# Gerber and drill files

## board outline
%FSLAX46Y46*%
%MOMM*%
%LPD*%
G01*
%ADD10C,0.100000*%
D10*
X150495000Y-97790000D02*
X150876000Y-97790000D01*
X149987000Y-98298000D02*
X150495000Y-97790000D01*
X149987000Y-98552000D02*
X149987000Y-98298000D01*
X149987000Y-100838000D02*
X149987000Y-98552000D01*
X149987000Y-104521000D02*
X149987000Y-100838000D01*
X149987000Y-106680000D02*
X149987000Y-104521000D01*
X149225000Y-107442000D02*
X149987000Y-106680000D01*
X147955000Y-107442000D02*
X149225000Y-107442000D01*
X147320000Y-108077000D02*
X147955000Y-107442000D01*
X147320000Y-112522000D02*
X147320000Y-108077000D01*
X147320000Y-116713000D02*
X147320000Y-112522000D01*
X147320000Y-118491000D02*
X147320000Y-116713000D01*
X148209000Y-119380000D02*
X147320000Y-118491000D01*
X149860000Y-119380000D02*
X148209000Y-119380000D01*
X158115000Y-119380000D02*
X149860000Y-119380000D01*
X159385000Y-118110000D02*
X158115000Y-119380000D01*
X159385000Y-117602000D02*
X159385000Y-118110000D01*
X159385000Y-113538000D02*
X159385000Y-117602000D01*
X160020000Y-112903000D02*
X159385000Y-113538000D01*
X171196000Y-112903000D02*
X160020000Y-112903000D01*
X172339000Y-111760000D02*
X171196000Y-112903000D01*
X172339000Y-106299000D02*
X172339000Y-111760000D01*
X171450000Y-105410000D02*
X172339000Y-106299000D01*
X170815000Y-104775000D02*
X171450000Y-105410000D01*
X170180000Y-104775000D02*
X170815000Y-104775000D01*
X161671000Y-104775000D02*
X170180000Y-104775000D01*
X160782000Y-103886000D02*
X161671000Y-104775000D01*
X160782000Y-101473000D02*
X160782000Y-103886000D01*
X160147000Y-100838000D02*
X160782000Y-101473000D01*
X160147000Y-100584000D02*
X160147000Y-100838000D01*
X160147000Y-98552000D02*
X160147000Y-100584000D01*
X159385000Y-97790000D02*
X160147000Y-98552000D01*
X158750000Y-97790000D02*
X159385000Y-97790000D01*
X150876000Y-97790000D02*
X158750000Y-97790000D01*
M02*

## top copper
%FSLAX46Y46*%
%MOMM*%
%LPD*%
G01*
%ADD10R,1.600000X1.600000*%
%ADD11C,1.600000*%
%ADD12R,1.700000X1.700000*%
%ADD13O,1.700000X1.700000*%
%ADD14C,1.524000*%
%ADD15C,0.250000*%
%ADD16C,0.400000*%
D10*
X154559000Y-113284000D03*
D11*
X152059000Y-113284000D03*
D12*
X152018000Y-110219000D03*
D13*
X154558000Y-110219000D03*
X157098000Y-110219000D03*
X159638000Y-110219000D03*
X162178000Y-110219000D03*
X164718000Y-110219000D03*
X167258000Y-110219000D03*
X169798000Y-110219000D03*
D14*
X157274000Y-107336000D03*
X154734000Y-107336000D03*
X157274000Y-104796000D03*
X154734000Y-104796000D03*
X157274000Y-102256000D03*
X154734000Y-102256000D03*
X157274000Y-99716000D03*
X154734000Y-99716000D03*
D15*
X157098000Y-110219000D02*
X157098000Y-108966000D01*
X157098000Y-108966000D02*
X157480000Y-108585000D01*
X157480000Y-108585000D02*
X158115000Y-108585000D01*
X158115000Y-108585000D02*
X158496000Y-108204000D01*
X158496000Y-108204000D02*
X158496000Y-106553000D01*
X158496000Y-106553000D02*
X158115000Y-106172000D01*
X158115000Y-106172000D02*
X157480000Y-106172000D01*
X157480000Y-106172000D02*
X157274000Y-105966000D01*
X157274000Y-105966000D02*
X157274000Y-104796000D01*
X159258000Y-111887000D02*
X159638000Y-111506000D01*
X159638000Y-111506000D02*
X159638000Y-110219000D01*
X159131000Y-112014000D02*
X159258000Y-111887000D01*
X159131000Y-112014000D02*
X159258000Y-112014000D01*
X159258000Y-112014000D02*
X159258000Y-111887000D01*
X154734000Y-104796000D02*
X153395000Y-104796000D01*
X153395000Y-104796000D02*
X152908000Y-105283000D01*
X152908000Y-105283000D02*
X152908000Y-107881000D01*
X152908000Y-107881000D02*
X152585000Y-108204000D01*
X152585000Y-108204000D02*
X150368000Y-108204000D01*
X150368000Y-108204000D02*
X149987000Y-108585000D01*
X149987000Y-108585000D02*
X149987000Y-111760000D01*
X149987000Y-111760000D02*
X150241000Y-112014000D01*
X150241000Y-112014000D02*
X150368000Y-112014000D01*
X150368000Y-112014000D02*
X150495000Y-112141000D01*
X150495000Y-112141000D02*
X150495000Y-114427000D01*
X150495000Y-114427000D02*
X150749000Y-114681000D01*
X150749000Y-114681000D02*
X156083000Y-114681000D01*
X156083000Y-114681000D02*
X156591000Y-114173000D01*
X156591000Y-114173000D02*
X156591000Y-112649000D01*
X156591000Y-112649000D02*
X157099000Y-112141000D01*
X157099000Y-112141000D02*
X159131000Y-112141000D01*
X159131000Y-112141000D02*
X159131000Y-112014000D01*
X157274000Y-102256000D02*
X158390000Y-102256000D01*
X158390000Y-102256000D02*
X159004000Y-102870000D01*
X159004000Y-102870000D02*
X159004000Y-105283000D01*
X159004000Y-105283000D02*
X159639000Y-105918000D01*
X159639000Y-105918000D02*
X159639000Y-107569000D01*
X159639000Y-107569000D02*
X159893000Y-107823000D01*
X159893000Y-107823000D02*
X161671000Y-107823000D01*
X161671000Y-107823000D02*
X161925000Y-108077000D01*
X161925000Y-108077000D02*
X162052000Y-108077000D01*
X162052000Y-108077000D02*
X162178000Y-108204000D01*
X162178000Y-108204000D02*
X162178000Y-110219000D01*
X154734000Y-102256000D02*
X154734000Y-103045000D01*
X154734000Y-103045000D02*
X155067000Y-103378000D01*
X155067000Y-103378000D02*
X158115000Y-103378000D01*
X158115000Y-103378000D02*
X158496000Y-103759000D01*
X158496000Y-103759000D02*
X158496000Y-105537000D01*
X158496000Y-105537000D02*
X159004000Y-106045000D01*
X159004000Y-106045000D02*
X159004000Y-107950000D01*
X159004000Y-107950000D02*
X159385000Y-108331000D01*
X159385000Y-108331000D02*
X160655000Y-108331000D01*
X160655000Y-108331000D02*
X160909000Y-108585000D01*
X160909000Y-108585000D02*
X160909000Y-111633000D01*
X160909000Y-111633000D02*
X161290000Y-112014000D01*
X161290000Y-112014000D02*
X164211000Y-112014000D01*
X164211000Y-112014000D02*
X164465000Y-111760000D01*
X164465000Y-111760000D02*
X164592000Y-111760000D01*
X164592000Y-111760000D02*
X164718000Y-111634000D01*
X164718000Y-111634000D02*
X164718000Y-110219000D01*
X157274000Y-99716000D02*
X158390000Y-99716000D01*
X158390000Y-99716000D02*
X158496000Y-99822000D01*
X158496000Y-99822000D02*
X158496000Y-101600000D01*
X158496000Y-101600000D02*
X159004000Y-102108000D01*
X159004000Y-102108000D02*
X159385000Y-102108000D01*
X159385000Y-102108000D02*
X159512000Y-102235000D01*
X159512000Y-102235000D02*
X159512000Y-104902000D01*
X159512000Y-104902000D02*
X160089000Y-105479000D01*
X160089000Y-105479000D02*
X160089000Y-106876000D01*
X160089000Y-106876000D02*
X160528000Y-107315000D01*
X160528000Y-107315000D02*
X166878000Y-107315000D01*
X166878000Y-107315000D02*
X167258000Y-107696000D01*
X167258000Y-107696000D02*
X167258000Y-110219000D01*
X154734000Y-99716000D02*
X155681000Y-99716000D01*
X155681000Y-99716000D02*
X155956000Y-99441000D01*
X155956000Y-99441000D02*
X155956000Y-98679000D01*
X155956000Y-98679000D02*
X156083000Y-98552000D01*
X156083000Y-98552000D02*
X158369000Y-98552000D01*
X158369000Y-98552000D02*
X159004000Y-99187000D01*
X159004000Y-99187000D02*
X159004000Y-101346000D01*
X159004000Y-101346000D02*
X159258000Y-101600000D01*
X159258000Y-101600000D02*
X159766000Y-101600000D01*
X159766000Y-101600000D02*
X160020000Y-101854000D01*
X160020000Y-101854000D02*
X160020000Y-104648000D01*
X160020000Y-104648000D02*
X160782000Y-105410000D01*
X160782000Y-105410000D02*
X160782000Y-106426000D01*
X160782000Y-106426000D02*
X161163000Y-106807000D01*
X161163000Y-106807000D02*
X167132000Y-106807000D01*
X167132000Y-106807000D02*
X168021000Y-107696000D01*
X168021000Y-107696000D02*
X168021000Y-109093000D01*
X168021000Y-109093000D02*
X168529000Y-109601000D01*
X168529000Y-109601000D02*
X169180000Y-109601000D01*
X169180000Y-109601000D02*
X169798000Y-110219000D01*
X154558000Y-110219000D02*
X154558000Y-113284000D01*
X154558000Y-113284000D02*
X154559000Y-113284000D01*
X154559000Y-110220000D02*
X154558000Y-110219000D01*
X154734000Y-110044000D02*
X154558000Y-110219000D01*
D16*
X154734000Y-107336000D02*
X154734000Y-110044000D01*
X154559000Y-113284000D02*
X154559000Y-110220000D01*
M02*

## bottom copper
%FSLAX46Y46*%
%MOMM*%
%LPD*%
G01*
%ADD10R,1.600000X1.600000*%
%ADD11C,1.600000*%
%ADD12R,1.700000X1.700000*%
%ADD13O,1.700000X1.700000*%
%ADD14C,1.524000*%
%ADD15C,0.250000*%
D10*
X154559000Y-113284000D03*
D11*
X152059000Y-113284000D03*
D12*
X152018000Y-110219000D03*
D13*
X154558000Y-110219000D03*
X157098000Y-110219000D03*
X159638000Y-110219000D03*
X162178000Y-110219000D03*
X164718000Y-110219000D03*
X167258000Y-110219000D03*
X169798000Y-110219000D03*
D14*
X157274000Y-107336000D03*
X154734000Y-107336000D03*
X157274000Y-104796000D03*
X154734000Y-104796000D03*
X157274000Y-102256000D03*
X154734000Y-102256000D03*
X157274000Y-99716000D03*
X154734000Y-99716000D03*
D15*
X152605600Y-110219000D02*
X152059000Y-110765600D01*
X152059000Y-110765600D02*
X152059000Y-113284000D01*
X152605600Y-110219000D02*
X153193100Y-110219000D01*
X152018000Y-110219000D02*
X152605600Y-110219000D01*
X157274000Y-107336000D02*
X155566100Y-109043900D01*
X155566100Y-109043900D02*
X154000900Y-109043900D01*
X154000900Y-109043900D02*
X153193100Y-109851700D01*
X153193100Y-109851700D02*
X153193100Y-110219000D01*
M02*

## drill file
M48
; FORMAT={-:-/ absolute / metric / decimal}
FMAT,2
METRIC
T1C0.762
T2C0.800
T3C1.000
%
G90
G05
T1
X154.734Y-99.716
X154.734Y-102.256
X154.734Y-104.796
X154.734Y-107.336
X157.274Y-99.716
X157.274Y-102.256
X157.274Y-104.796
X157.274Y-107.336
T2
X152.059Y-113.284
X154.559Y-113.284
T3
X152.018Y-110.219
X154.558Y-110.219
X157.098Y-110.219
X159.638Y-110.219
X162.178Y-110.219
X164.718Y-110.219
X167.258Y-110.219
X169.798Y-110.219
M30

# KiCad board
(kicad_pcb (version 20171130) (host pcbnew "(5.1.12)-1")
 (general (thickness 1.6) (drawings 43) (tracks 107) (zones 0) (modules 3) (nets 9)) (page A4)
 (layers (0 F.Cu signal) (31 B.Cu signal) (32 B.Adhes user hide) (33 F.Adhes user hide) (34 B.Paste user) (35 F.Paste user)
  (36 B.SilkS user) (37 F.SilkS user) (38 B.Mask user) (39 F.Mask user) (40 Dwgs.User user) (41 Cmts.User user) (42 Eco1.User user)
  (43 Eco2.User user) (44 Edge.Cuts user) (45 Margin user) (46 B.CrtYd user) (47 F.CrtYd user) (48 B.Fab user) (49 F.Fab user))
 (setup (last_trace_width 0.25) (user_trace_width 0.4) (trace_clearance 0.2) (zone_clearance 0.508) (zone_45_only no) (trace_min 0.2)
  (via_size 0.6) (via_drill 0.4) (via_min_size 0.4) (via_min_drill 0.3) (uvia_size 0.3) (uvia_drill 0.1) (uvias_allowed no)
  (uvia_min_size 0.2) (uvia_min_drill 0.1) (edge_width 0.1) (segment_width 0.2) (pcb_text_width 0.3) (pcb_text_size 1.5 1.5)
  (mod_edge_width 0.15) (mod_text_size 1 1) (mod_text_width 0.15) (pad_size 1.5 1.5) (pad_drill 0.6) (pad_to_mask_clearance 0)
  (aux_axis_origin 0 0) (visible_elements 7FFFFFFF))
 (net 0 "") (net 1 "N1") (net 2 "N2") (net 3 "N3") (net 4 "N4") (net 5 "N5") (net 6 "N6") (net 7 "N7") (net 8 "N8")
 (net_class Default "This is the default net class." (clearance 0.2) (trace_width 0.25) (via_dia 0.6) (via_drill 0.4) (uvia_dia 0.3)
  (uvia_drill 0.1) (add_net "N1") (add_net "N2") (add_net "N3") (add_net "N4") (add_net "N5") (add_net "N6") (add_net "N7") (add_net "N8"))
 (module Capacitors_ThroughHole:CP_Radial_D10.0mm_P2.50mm (layer F.Cu) (at 154.559 113.284 180)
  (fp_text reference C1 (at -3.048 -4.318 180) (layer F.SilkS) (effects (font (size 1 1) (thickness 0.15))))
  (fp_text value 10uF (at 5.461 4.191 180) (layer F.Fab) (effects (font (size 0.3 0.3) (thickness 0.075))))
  (pad 1 thru_hole rect (at 0 0 180) (size 1.6 1.6) (drill 0.8) (layers *.Cu *.Mask) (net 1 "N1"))
  (pad 2 thru_hole circle (at 2.5 0 180) (size 1.6 1.6) (drill 0.8) (layers *.Cu *.Mask) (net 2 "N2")))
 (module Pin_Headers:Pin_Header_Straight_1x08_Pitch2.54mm (layer F.Cu) (at 152.018 110.219 90)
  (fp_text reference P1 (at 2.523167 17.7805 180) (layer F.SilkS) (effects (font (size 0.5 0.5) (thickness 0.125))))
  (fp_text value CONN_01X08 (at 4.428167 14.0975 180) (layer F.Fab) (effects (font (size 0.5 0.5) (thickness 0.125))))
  (pad 1 thru_hole rect (at 0 0 90) (size 1.7 1.7) (drill 1) (layers *.Cu *.Mask) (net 2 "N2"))
  (pad 2 thru_hole oval (at 0 2.54 90) (size 1.7 1.7) (drill 1) (layers *.Cu *.Mask) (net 1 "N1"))
  (pad 3 thru_hole oval (at 0 5.08 90) (size 1.7 1.7) (drill 1) (layers *.Cu *.Mask) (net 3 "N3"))
  (pad 4 thru_hole oval (at 0 7.62 90) (size 1.7 1.7) (drill 1) (layers *.Cu *.Mask) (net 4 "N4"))
  (pad 5 thru_hole oval (at 0 10.16 90) (size 1.7 1.7) (drill 1) (layers *.Cu *.Mask) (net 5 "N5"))
  (pad 6 thru_hole oval (at 0 12.7 90) (size 1.7 1.7) (drill 1) (layers *.Cu *.Mask) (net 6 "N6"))
  (pad 7 thru_hole oval (at 0 15.24 90) (size 1.7 1.7) (drill 1) (layers *.Cu *.Mask) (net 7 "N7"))
  (pad 8 thru_hole oval (at 0 17.78 90) (size 1.7 1.7) (drill 1) (layers *.Cu *.Mask) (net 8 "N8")))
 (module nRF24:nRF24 (layer F.Cu) (at 154.734 103.78)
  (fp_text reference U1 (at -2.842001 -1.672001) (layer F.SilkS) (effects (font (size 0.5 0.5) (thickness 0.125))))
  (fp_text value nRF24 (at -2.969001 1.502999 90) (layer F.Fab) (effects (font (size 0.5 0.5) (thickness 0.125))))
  (pad 1 thru_hole circle (at 2.54 3.556) (size 1.524 1.524) (drill 0.762) (layers *.Cu *.Mask) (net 2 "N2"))
  (pad 2 thru_hole circle (at 0 3.556) (size 1.524 1.524) (drill 0.762) (layers *.Cu *.Mask) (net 1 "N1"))
  (pad 3 thru_hole circle (at 2.54 1.016) (size 1.524 1.524) (drill 0.762) (layers *.Cu *.Mask) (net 3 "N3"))
  (pad 4 thru_hole circle (at 0 1.016) (size 1.524 1.524) (drill 0.762) (layers *.Cu *.Mask) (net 4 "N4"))
  (pad 5 thru_hole circle (at 2.54 -1.524) (size 1.524 1.524) (drill 0.762) (layers *.Cu *.Mask) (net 5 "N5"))
  (pad 6 thru_hole circle (at 0 -1.524) (size 1.524 1.524) (drill 0.762) (layers *.Cu *.Mask) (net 6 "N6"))
  (pad 7 thru_hole circle (at 2.54 -4.064) (size 1.524 1.524) (drill 0.762) (layers *.Cu *.Mask) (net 7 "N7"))
  (pad 8 thru_hole circle (at 0 -4.064) (size 1.524 1.524) (drill 0.762) (layers *.Cu *.Mask) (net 8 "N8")))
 (gr_line (start 150.495 97.79) (end 150.876 97.79) (angle 90) (layer Edge.Cuts) (width 0.1))
 (gr_line (start 149.987 98.298) (end 150.495 97.79) (angle 90) (layer Edge.Cuts) (width 0.1))
 (gr_line (start 149.987 98.552) (end 149.987 98.298) (angle 90) (layer Edge.Cuts) (width 0.1))
 (gr_line (start 149.987 100.838) (end 149.987 98.552) (angle 90) (layer Edge.Cuts) (width 0.1))
 (gr_line (start 149.987 104.521) (end 149.987 100.838) (angle 90) (layer Edge.Cuts) (width 0.1))
 (gr_line (start 149.987 106.68) (end 149.987 104.521) (angle 90) (layer Edge.Cuts) (width 0.1))
 (gr_line (start 149.225 107.442) (end 149.987 106.68) (angle 90) (layer Edge.Cuts) (width 0.1))
 (gr_line (start 147.955 107.442) (end 149.225 107.442) (angle 90) (layer Edge.Cuts) (width 0.1))
 (gr_line (start 147.32 108.077) (end 147.955 107.442) (angle 90) (layer Edge.Cuts) (width 0.1))
 (gr_line (start 147.32 112.522) (end 147.32 108.077) (angle 90) (layer Edge.Cuts) (width 0.1))
 (gr_line (start 147.32 116.713) (end 147.32 112.522) (angle 90) (layer Edge.Cuts) (width 0.1))
 (gr_line (start 147.32 118.491) (end 147.32 116.713) (angle 90) (layer Edge.Cuts) (width 0.1))
 (gr_line (start 148.209 119.38) (end 147.32 118.491) (angle 90) (layer Edge.Cuts) (width 0.1))
 (gr_line (start 149.86 119.38) (end 148.209 119.38) (angle 90) (layer Edge.Cuts) (width 0.1))
 (gr_line (start 158.115 119.38) (end 149.86 119.38) (angle 90) (layer Edge.Cuts) (width 0.1))
 (gr_line (start 159.385 118.11) (end 158.115 119.38) (angle 90) (layer Edge.Cuts) (width 0.1))
 (gr_line (start 159.385 117.602) (end 159.385 118.11) (angle 90) (layer Edge.Cuts) (width 0.1))
 (gr_line (start 159.385 113.538) (end 159.385 117.602) (angle 90) (layer Edge.Cuts) (width 0.1))
 (gr_line (start 160.02 112.903) (end 159.385 113.538) (angle 90) (layer Edge.Cuts) (width 0.1))
 (gr_line (start 171.196 112.903) (end 160.02 112.903) (angle 90) (layer Edge.Cuts) (width 0.1))
 (gr_line (start 172.339 111.76) (end 171.196 112.903) (angle 90) (layer Edge.Cuts) (width 0.1))
 (gr_line (start 172.339 106.299) (end 172.339 111.76) (angle 90) (layer Edge.Cuts) (width 0.1))
 (gr_line (start 171.45 105.41) (end 172.339 106.299) (angle 90) (layer Edge.Cuts) (width 0.1))
 (gr_line (start 170.815 104.775) (end 171.45 105.41) (angle 90) (layer Edge.Cuts) (width 0.1))
 (gr_line (start 170.18 104.775) (end 170.815 104.775) (angle 90) (layer Edge.Cuts) (width 0.1))
 (gr_line (start 161.671 104.775) (end 170.18 104.775) (angle 90) (layer Edge.Cuts) (width 0.1))
 (gr_line (start 160.782 103.886) (end 161.671 104.775) (angle 90) (layer Edge.Cuts) (width 0.1))
 (gr_line (start 160.782 101.473) (end 160.782 103.886) (angle 90) (layer Edge.Cuts) (width 0.1))
 (gr_line (start 160.147 100.838) (end 160.782 101.473) (angle 90) (layer Edge.Cuts) (width 0.1))
 (gr_line (start 160.147 100.584) (end 160.147 100.838) (angle 90) (layer Edge.Cuts) (width 0.1))
 (gr_line (start 160.147 98.552) (end 160.147 100.584) (angle 90) (layer Edge.Cuts) (width 0.1))
 (gr_line (start 159.385 97.79) (end 160.147 98.552) (angle 90) (layer Edge.Cuts) (width 0.1))
 (gr_line (start 158.75 97.79) (end 159.385 97.79) (angle 90) (layer Edge.Cuts) (width 0.1))
 (gr_line (start 150.876 97.79) (end 158.75 97.79) (angle 90) (layer Edge.Cuts) (width 0.1))
 (segment (start 157.098 110.219) (end 157.098 108.966) (width 0.25) (layer F.Cu) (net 3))
 (segment (start 157.098 108.966) (end 157.48 108.585) (width 0.25) (layer F.Cu) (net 3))
 (segment (start 157.48 108.585) (end 158.115 108.585) (width 0.25) (layer F.Cu) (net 3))
 (segment (start 158.115 108.585) (end 158.496 108.204) (width 0.25) (layer F.Cu) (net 3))
 (segment (start 158.496 108.204) (end 158.496 106.553) (width 0.25) (layer F.Cu) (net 3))
 (segment (start 158.496 106.553) (end 158.115 106.172) (width 0.25) (layer F.Cu) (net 3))
 (segment (start 158.115 106.172) (end 157.48 106.172) (width 0.25) (layer F.Cu) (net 3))
 (segment (start 157.48 106.172) (end 157.274 105.966) (width 0.25) (layer F.Cu) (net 3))
 (segment (start 157.274 105.966) (end 157.274 104.796) (width 0.25) (layer F.Cu) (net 3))
 (segment (start 159.258 111.887) (end 159.638 111.506) (width 0.25) (layer F.Cu) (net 4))
 (segment (start 159.638 111.506) (end 159.638 110.219) (width 0.25) (layer F.Cu) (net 4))
 (segment (start 159.131 112.014) (end 159.258 111.887) (width 0.25) (layer F.Cu) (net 4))
 (segment (start 159.131 112.014) (end 159.258 112.014) (width 0.25) (layer F.Cu) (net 4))
 (segment (start 159.258 112.014) (end 159.258 111.887) (width 0.25) (layer F.Cu) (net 4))
 (segment (start 154.734 104.796) (end 153.395 104.796) (width 0.25) (layer F.Cu) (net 4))
 (segment (start 153.395 104.796) (end 152.908 105.283) (width 0.25) (layer F.Cu) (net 4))
 (segment (start 152.908 105.283) (end 152.908 107.881) (width 0.25) (layer F.Cu) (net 4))
 (segment (start 152.908 107.881) (end 152.585 108.204) (width 0.25) (layer F.Cu) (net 4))
 (segment (start 152.585 108.204) (end 150.368 108.204) (width 0.25) (layer F.Cu) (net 4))
 (segment (start 150.368 108.204) (end 149.987 108.585) (width 0.25) (layer F.Cu) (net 4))
 (segment (start 149.987 108.585) (end 149.987 111.76) (width 0.25) (layer F.Cu) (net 4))
 (segment (start 149.987 111.76) (end 150.241 112.014) (width 0.25) (layer F.Cu) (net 4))
 (segment (start 150.241 112.014) (end 150.368 112.014) (width 0.25) (layer F.Cu) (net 4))
 (segment (start 150.368 112.014) (end 150.495 112.141) (width 0.25) (layer F.Cu) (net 4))
 (segment (start 150.495 112.141) (end 150.495 114.427) (width 0.25) (layer F.Cu) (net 4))
 (segment (start 150.495 114.427) (end 150.749 114.681) (width 0.25) (layer F.Cu) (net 4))
 (segment (start 150.749 114.681) (end 156.083 114.681) (width 0.25) (layer F.Cu) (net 4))
 (segment (start 156.083 114.681) (end 156.591 114.173) (width 0.25) (layer F.Cu) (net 4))
 (segment (start 156.591 114.173) (end 156.591 112.649) (width 0.25) (layer F.Cu) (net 4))
 (segment (start 156.591 112.649) (end 157.099 112.141) (width 0.25) (layer F.Cu) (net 4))
 (segment (start 157.099 112.141) (end 159.131 112.141) (width 0.25) (layer F.Cu) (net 4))
 (segment (start 159.131 112.141) (end 159.131 112.014) (width 0.25) (layer F.Cu) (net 4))
 (segment (start 157.274 102.256) (end 158.39 102.256) (width 0.25) (layer F.Cu) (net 5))
 (segment (start 158.39 102.256) (end 159.004 102.87) (width 0.25) (layer F.Cu) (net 5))
 (segment (start 159.004 102.87) (end 159.004 105.283) (width 0.25) (layer F.Cu) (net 5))
 (segment (start 159.004 105.283) (end 159.639 105.918) (width 0.25) (layer F.Cu) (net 5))
 (segment (start 159.639 105.918) (end 159.639 107.569) (width 0.25) (layer F.Cu) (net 5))
 (segment (start 159.639 107.569) (end 159.893 107.823) (width 0.25) (layer F.Cu) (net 5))
 (segment (start 159.893 107.823) (end 161.671 107.823) (width 0.25) (layer F.Cu) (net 5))
 (segment (start 161.671 107.823) (end 161.925 108.077) (width 0.25) (layer F.Cu) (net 5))
 (segment (start 161.925 108.077) (end 162.052 108.077) (width 0.25) (layer F.Cu) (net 5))
 (segment (start 162.052 108.077) (end 162.178 108.204) (width 0.25) (layer F.Cu) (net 5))
 (segment (start 162.178 108.204) (end 162.178 110.219) (width 0.25) (layer F.Cu) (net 5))
 (segment (start 154.734 102.256) (end 154.734 103.045) (width 0.25) (layer F.Cu) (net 6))
 (segment (start 154.734 103.045) (end 155.067 103.378) (width 0.25) (layer F.Cu) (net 6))
 (segment (start 155.067 103.378) (end 158.115 103.378) (width 0.25) (layer F.Cu) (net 6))
 (segment (start 158.115 103.378) (end 158.496 103.759) (width 0.25) (layer F.Cu) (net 6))
 (segment (start 158.496 103.759) (end 158.496 105.537) (width 0.25) (layer F.Cu) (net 6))
 (segment (start 158.496 105.537) (end 159.004 106.045) (width 0.25) (layer F.Cu) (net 6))
 (segment (start 159.004 106.045) (end 159.004 107.95) (width 0.25) (layer F.Cu) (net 6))
 (segment (start 159.004 107.95) (end 159.385 108.331) (width 0.25) (layer F.Cu) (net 6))
 (segment (start 159.385 108.331) (end 160.655 108.331) (width 0.25) (layer F.Cu) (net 6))
 (segment (start 160.655 108.331) (end 160.909 108.585) (width 0.25) (layer F.Cu) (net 6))
 (segment (start 160.909 108.585) (end 160.909 111.633) (width 0.25) (layer F.Cu) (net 6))
 (segment (start 160.909 111.633) (end 161.29 112.014) (width 0.25) (layer F.Cu) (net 6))
 (segment (start 161.29 112.014) (end 164.211 112.014) (width 0.25) (layer F.Cu) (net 6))
 (segment (start 164.211 112.014) (end 164.465 111.76) (width 0.25) (layer F.Cu) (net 6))
 (segment (start 164.465 111.76) (end 164.592 111.76) (width 0.25) (layer F.Cu) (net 6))
 (segment (start 164.592 111.76) (end 164.718 111.634) (width 0.25) (layer F.Cu) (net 6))
 (segment (start 164.718 111.634) (end 164.718 110.219) (width 0.25) (layer F.Cu) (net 6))
 (segment (start 157.274 99.716) (end 158.39 99.716) (width 0.25) (layer F.Cu) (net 7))
 (segment (start 158.39 99.716) (end 158.496 99.822) (width 0.25) (layer F.Cu) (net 7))
 (segment (start 158.496 99.822) (end 158.496 101.6) (width 0.25) (layer F.Cu) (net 7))
 (segment (start 158.496 101.6) (end 159.004 102.108) (width 0.25) (layer F.Cu) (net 7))
 (segment (start 159.004 102.108) (end 159.385 102.108) (width 0.25) (layer F.Cu) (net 7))
 (segment (start 159.385 102.108) (end 159.512 102.235) (width 0.25) (layer F.Cu) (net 7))
 (segment (start 159.512 102.235) (end 159.512 104.902) (width 0.25) (layer F.Cu) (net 7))
 (segment (start 159.512 104.902) (end 160.089 105.479) (width 0.25) (layer F.Cu) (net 7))
 (segment (start 160.089 105.479) (end 160.089 106.876) (width 0.25) (layer F.Cu) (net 7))
 (segment (start 160.089 106.876) (end 160.528 107.315) (width 0.25) (layer F.Cu) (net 7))
 (segment (start 160.528 107.315) (end 166.878 107.315) (width 0.25) (layer F.Cu) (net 7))
 (segment (start 166.878 107.315) (end 167.258 107.696) (width 0.25) (layer F.Cu) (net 7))
 (segment (start 167.258 107.696) (end 167.258 110.219) (width 0.25) (layer F.Cu) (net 7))
 (segment (start 154.734 99.716) (end 155.681 99.716) (width 0.25) (layer F.Cu) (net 8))
 (segment (start 155.681 99.716) (end 155.956 99.441) (width 0.25) (layer F.Cu) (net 8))
 (segment (start 155.956 99.441) (end 155.956 98.679) (width 0.25) (layer F.Cu) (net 8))
 (segment (start 155.956 98.679) (end 156.083 98.552) (width 0.25) (layer F.Cu) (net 8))
 (segment (start 156.083 98.552) (end 158.369 98.552) (width 0.25) (layer F.Cu) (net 8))
 (segment (start 158.369 98.552) (end 159.004 99.187) (width 0.25) (layer F.Cu) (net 8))
 (segment (start 159.004 99.187) (end 159.004 101.346) (width 0.25) (layer F.Cu) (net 8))
 (segment (start 159.004 101.346) (end 159.258 101.6) (width 0.25) (layer F.Cu) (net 8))
 (segment (start 159.258 101.6) (end 159.766 101.6) (width 0.25) (layer F.Cu) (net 8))
 (segment (start 159.766 101.6) (end 160.02 101.854) (width 0.25) (layer F.Cu) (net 8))
 (segment (start 160.02 101.854) (end 160.02 104.648) (width 0.25) (layer F.Cu) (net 8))
 (segment (start 160.02 104.648) (end 160.782 105.41) (width 0.25) (layer F.Cu) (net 8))
 (segment (start 160.782 105.41) (end 160.782 106.426) (width 0.25) (layer F.Cu) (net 8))
 (segment (start 160.782 106.426) (end 161.163 106.807) (width 0.25) (layer F.Cu) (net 8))
 (segment (start 161.163 106.807) (end 167.132 106.807) (width 0.25) (layer F.Cu) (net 8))
 (segment (start 167.132 106.807) (end 168.021 107.696) (width 0.25) (layer F.Cu) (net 8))
 (segment (start 168.021 107.696) (end 168.021 109.093) (width 0.25) (layer F.Cu) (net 8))
 (segment (start 168.021 109.093) (end 168.529 109.601) (width 0.25) (layer F.Cu) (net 8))
 (segment (start 168.529 109.601) (end 169.18 109.601) (width 0.25) (layer F.Cu) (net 8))
 (segment (start 169.18 109.601) (end 169.798 110.219) (width 0.25) (layer F.Cu) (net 8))
 (segment (start 154.558 110.219) (end 154.558 113.284) (width 0.25) (layer F.Cu) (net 1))
 (segment (start 154.558 113.284) (end 154.559 113.284) (width 0.25) (layer F.Cu) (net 1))
 (segment (start 154.559 110.22) (end 154.558 110.219) (width 0.25) (layer F.Cu) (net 1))
 (segment (start 154.734 110.044) (end 154.558 110.219) (width 0.25) (layer F.Cu) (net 1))
 (segment (start 154.734 107.336) (end 154.734 110.044) (width 0.4) (layer F.Cu) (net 1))
 (segment (start 154.559 113.284) (end 154.559 110.22) (width 0.4) (layer F.Cu) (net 1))
 (segment (start 152.6056 110.219) (end 152.059 110.7656) (width 0.25) (layer B.Cu) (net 2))
 (segment (start 152.059 110.7656) (end 152.059 113.284) (width 0.25) (layer B.Cu) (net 2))
 (segment (start 152.6056 110.219) (end 153.1931 110.219) (width 0.25) (layer B.Cu) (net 2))
 (segment (start 152.018 110.219) (end 152.6056 110.219) (width 0.25) (layer B.Cu) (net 2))
 (segment (start 157.274 107.336) (end 155.5661 109.0439) (width 0.25) (layer B.Cu) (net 2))
 (segment (start 155.5661 109.0439) (end 154.0009 109.0439) (width 0.25) (layer B.Cu) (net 2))
 (segment (start 154.0009 109.0439) (end 153.1931 109.8517) (width 0.25) (layer B.Cu) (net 2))
 (segment (start 153.1931 109.8517) (end 153.1931 110.219) (width 0.25) (layer B.Cu) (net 2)))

